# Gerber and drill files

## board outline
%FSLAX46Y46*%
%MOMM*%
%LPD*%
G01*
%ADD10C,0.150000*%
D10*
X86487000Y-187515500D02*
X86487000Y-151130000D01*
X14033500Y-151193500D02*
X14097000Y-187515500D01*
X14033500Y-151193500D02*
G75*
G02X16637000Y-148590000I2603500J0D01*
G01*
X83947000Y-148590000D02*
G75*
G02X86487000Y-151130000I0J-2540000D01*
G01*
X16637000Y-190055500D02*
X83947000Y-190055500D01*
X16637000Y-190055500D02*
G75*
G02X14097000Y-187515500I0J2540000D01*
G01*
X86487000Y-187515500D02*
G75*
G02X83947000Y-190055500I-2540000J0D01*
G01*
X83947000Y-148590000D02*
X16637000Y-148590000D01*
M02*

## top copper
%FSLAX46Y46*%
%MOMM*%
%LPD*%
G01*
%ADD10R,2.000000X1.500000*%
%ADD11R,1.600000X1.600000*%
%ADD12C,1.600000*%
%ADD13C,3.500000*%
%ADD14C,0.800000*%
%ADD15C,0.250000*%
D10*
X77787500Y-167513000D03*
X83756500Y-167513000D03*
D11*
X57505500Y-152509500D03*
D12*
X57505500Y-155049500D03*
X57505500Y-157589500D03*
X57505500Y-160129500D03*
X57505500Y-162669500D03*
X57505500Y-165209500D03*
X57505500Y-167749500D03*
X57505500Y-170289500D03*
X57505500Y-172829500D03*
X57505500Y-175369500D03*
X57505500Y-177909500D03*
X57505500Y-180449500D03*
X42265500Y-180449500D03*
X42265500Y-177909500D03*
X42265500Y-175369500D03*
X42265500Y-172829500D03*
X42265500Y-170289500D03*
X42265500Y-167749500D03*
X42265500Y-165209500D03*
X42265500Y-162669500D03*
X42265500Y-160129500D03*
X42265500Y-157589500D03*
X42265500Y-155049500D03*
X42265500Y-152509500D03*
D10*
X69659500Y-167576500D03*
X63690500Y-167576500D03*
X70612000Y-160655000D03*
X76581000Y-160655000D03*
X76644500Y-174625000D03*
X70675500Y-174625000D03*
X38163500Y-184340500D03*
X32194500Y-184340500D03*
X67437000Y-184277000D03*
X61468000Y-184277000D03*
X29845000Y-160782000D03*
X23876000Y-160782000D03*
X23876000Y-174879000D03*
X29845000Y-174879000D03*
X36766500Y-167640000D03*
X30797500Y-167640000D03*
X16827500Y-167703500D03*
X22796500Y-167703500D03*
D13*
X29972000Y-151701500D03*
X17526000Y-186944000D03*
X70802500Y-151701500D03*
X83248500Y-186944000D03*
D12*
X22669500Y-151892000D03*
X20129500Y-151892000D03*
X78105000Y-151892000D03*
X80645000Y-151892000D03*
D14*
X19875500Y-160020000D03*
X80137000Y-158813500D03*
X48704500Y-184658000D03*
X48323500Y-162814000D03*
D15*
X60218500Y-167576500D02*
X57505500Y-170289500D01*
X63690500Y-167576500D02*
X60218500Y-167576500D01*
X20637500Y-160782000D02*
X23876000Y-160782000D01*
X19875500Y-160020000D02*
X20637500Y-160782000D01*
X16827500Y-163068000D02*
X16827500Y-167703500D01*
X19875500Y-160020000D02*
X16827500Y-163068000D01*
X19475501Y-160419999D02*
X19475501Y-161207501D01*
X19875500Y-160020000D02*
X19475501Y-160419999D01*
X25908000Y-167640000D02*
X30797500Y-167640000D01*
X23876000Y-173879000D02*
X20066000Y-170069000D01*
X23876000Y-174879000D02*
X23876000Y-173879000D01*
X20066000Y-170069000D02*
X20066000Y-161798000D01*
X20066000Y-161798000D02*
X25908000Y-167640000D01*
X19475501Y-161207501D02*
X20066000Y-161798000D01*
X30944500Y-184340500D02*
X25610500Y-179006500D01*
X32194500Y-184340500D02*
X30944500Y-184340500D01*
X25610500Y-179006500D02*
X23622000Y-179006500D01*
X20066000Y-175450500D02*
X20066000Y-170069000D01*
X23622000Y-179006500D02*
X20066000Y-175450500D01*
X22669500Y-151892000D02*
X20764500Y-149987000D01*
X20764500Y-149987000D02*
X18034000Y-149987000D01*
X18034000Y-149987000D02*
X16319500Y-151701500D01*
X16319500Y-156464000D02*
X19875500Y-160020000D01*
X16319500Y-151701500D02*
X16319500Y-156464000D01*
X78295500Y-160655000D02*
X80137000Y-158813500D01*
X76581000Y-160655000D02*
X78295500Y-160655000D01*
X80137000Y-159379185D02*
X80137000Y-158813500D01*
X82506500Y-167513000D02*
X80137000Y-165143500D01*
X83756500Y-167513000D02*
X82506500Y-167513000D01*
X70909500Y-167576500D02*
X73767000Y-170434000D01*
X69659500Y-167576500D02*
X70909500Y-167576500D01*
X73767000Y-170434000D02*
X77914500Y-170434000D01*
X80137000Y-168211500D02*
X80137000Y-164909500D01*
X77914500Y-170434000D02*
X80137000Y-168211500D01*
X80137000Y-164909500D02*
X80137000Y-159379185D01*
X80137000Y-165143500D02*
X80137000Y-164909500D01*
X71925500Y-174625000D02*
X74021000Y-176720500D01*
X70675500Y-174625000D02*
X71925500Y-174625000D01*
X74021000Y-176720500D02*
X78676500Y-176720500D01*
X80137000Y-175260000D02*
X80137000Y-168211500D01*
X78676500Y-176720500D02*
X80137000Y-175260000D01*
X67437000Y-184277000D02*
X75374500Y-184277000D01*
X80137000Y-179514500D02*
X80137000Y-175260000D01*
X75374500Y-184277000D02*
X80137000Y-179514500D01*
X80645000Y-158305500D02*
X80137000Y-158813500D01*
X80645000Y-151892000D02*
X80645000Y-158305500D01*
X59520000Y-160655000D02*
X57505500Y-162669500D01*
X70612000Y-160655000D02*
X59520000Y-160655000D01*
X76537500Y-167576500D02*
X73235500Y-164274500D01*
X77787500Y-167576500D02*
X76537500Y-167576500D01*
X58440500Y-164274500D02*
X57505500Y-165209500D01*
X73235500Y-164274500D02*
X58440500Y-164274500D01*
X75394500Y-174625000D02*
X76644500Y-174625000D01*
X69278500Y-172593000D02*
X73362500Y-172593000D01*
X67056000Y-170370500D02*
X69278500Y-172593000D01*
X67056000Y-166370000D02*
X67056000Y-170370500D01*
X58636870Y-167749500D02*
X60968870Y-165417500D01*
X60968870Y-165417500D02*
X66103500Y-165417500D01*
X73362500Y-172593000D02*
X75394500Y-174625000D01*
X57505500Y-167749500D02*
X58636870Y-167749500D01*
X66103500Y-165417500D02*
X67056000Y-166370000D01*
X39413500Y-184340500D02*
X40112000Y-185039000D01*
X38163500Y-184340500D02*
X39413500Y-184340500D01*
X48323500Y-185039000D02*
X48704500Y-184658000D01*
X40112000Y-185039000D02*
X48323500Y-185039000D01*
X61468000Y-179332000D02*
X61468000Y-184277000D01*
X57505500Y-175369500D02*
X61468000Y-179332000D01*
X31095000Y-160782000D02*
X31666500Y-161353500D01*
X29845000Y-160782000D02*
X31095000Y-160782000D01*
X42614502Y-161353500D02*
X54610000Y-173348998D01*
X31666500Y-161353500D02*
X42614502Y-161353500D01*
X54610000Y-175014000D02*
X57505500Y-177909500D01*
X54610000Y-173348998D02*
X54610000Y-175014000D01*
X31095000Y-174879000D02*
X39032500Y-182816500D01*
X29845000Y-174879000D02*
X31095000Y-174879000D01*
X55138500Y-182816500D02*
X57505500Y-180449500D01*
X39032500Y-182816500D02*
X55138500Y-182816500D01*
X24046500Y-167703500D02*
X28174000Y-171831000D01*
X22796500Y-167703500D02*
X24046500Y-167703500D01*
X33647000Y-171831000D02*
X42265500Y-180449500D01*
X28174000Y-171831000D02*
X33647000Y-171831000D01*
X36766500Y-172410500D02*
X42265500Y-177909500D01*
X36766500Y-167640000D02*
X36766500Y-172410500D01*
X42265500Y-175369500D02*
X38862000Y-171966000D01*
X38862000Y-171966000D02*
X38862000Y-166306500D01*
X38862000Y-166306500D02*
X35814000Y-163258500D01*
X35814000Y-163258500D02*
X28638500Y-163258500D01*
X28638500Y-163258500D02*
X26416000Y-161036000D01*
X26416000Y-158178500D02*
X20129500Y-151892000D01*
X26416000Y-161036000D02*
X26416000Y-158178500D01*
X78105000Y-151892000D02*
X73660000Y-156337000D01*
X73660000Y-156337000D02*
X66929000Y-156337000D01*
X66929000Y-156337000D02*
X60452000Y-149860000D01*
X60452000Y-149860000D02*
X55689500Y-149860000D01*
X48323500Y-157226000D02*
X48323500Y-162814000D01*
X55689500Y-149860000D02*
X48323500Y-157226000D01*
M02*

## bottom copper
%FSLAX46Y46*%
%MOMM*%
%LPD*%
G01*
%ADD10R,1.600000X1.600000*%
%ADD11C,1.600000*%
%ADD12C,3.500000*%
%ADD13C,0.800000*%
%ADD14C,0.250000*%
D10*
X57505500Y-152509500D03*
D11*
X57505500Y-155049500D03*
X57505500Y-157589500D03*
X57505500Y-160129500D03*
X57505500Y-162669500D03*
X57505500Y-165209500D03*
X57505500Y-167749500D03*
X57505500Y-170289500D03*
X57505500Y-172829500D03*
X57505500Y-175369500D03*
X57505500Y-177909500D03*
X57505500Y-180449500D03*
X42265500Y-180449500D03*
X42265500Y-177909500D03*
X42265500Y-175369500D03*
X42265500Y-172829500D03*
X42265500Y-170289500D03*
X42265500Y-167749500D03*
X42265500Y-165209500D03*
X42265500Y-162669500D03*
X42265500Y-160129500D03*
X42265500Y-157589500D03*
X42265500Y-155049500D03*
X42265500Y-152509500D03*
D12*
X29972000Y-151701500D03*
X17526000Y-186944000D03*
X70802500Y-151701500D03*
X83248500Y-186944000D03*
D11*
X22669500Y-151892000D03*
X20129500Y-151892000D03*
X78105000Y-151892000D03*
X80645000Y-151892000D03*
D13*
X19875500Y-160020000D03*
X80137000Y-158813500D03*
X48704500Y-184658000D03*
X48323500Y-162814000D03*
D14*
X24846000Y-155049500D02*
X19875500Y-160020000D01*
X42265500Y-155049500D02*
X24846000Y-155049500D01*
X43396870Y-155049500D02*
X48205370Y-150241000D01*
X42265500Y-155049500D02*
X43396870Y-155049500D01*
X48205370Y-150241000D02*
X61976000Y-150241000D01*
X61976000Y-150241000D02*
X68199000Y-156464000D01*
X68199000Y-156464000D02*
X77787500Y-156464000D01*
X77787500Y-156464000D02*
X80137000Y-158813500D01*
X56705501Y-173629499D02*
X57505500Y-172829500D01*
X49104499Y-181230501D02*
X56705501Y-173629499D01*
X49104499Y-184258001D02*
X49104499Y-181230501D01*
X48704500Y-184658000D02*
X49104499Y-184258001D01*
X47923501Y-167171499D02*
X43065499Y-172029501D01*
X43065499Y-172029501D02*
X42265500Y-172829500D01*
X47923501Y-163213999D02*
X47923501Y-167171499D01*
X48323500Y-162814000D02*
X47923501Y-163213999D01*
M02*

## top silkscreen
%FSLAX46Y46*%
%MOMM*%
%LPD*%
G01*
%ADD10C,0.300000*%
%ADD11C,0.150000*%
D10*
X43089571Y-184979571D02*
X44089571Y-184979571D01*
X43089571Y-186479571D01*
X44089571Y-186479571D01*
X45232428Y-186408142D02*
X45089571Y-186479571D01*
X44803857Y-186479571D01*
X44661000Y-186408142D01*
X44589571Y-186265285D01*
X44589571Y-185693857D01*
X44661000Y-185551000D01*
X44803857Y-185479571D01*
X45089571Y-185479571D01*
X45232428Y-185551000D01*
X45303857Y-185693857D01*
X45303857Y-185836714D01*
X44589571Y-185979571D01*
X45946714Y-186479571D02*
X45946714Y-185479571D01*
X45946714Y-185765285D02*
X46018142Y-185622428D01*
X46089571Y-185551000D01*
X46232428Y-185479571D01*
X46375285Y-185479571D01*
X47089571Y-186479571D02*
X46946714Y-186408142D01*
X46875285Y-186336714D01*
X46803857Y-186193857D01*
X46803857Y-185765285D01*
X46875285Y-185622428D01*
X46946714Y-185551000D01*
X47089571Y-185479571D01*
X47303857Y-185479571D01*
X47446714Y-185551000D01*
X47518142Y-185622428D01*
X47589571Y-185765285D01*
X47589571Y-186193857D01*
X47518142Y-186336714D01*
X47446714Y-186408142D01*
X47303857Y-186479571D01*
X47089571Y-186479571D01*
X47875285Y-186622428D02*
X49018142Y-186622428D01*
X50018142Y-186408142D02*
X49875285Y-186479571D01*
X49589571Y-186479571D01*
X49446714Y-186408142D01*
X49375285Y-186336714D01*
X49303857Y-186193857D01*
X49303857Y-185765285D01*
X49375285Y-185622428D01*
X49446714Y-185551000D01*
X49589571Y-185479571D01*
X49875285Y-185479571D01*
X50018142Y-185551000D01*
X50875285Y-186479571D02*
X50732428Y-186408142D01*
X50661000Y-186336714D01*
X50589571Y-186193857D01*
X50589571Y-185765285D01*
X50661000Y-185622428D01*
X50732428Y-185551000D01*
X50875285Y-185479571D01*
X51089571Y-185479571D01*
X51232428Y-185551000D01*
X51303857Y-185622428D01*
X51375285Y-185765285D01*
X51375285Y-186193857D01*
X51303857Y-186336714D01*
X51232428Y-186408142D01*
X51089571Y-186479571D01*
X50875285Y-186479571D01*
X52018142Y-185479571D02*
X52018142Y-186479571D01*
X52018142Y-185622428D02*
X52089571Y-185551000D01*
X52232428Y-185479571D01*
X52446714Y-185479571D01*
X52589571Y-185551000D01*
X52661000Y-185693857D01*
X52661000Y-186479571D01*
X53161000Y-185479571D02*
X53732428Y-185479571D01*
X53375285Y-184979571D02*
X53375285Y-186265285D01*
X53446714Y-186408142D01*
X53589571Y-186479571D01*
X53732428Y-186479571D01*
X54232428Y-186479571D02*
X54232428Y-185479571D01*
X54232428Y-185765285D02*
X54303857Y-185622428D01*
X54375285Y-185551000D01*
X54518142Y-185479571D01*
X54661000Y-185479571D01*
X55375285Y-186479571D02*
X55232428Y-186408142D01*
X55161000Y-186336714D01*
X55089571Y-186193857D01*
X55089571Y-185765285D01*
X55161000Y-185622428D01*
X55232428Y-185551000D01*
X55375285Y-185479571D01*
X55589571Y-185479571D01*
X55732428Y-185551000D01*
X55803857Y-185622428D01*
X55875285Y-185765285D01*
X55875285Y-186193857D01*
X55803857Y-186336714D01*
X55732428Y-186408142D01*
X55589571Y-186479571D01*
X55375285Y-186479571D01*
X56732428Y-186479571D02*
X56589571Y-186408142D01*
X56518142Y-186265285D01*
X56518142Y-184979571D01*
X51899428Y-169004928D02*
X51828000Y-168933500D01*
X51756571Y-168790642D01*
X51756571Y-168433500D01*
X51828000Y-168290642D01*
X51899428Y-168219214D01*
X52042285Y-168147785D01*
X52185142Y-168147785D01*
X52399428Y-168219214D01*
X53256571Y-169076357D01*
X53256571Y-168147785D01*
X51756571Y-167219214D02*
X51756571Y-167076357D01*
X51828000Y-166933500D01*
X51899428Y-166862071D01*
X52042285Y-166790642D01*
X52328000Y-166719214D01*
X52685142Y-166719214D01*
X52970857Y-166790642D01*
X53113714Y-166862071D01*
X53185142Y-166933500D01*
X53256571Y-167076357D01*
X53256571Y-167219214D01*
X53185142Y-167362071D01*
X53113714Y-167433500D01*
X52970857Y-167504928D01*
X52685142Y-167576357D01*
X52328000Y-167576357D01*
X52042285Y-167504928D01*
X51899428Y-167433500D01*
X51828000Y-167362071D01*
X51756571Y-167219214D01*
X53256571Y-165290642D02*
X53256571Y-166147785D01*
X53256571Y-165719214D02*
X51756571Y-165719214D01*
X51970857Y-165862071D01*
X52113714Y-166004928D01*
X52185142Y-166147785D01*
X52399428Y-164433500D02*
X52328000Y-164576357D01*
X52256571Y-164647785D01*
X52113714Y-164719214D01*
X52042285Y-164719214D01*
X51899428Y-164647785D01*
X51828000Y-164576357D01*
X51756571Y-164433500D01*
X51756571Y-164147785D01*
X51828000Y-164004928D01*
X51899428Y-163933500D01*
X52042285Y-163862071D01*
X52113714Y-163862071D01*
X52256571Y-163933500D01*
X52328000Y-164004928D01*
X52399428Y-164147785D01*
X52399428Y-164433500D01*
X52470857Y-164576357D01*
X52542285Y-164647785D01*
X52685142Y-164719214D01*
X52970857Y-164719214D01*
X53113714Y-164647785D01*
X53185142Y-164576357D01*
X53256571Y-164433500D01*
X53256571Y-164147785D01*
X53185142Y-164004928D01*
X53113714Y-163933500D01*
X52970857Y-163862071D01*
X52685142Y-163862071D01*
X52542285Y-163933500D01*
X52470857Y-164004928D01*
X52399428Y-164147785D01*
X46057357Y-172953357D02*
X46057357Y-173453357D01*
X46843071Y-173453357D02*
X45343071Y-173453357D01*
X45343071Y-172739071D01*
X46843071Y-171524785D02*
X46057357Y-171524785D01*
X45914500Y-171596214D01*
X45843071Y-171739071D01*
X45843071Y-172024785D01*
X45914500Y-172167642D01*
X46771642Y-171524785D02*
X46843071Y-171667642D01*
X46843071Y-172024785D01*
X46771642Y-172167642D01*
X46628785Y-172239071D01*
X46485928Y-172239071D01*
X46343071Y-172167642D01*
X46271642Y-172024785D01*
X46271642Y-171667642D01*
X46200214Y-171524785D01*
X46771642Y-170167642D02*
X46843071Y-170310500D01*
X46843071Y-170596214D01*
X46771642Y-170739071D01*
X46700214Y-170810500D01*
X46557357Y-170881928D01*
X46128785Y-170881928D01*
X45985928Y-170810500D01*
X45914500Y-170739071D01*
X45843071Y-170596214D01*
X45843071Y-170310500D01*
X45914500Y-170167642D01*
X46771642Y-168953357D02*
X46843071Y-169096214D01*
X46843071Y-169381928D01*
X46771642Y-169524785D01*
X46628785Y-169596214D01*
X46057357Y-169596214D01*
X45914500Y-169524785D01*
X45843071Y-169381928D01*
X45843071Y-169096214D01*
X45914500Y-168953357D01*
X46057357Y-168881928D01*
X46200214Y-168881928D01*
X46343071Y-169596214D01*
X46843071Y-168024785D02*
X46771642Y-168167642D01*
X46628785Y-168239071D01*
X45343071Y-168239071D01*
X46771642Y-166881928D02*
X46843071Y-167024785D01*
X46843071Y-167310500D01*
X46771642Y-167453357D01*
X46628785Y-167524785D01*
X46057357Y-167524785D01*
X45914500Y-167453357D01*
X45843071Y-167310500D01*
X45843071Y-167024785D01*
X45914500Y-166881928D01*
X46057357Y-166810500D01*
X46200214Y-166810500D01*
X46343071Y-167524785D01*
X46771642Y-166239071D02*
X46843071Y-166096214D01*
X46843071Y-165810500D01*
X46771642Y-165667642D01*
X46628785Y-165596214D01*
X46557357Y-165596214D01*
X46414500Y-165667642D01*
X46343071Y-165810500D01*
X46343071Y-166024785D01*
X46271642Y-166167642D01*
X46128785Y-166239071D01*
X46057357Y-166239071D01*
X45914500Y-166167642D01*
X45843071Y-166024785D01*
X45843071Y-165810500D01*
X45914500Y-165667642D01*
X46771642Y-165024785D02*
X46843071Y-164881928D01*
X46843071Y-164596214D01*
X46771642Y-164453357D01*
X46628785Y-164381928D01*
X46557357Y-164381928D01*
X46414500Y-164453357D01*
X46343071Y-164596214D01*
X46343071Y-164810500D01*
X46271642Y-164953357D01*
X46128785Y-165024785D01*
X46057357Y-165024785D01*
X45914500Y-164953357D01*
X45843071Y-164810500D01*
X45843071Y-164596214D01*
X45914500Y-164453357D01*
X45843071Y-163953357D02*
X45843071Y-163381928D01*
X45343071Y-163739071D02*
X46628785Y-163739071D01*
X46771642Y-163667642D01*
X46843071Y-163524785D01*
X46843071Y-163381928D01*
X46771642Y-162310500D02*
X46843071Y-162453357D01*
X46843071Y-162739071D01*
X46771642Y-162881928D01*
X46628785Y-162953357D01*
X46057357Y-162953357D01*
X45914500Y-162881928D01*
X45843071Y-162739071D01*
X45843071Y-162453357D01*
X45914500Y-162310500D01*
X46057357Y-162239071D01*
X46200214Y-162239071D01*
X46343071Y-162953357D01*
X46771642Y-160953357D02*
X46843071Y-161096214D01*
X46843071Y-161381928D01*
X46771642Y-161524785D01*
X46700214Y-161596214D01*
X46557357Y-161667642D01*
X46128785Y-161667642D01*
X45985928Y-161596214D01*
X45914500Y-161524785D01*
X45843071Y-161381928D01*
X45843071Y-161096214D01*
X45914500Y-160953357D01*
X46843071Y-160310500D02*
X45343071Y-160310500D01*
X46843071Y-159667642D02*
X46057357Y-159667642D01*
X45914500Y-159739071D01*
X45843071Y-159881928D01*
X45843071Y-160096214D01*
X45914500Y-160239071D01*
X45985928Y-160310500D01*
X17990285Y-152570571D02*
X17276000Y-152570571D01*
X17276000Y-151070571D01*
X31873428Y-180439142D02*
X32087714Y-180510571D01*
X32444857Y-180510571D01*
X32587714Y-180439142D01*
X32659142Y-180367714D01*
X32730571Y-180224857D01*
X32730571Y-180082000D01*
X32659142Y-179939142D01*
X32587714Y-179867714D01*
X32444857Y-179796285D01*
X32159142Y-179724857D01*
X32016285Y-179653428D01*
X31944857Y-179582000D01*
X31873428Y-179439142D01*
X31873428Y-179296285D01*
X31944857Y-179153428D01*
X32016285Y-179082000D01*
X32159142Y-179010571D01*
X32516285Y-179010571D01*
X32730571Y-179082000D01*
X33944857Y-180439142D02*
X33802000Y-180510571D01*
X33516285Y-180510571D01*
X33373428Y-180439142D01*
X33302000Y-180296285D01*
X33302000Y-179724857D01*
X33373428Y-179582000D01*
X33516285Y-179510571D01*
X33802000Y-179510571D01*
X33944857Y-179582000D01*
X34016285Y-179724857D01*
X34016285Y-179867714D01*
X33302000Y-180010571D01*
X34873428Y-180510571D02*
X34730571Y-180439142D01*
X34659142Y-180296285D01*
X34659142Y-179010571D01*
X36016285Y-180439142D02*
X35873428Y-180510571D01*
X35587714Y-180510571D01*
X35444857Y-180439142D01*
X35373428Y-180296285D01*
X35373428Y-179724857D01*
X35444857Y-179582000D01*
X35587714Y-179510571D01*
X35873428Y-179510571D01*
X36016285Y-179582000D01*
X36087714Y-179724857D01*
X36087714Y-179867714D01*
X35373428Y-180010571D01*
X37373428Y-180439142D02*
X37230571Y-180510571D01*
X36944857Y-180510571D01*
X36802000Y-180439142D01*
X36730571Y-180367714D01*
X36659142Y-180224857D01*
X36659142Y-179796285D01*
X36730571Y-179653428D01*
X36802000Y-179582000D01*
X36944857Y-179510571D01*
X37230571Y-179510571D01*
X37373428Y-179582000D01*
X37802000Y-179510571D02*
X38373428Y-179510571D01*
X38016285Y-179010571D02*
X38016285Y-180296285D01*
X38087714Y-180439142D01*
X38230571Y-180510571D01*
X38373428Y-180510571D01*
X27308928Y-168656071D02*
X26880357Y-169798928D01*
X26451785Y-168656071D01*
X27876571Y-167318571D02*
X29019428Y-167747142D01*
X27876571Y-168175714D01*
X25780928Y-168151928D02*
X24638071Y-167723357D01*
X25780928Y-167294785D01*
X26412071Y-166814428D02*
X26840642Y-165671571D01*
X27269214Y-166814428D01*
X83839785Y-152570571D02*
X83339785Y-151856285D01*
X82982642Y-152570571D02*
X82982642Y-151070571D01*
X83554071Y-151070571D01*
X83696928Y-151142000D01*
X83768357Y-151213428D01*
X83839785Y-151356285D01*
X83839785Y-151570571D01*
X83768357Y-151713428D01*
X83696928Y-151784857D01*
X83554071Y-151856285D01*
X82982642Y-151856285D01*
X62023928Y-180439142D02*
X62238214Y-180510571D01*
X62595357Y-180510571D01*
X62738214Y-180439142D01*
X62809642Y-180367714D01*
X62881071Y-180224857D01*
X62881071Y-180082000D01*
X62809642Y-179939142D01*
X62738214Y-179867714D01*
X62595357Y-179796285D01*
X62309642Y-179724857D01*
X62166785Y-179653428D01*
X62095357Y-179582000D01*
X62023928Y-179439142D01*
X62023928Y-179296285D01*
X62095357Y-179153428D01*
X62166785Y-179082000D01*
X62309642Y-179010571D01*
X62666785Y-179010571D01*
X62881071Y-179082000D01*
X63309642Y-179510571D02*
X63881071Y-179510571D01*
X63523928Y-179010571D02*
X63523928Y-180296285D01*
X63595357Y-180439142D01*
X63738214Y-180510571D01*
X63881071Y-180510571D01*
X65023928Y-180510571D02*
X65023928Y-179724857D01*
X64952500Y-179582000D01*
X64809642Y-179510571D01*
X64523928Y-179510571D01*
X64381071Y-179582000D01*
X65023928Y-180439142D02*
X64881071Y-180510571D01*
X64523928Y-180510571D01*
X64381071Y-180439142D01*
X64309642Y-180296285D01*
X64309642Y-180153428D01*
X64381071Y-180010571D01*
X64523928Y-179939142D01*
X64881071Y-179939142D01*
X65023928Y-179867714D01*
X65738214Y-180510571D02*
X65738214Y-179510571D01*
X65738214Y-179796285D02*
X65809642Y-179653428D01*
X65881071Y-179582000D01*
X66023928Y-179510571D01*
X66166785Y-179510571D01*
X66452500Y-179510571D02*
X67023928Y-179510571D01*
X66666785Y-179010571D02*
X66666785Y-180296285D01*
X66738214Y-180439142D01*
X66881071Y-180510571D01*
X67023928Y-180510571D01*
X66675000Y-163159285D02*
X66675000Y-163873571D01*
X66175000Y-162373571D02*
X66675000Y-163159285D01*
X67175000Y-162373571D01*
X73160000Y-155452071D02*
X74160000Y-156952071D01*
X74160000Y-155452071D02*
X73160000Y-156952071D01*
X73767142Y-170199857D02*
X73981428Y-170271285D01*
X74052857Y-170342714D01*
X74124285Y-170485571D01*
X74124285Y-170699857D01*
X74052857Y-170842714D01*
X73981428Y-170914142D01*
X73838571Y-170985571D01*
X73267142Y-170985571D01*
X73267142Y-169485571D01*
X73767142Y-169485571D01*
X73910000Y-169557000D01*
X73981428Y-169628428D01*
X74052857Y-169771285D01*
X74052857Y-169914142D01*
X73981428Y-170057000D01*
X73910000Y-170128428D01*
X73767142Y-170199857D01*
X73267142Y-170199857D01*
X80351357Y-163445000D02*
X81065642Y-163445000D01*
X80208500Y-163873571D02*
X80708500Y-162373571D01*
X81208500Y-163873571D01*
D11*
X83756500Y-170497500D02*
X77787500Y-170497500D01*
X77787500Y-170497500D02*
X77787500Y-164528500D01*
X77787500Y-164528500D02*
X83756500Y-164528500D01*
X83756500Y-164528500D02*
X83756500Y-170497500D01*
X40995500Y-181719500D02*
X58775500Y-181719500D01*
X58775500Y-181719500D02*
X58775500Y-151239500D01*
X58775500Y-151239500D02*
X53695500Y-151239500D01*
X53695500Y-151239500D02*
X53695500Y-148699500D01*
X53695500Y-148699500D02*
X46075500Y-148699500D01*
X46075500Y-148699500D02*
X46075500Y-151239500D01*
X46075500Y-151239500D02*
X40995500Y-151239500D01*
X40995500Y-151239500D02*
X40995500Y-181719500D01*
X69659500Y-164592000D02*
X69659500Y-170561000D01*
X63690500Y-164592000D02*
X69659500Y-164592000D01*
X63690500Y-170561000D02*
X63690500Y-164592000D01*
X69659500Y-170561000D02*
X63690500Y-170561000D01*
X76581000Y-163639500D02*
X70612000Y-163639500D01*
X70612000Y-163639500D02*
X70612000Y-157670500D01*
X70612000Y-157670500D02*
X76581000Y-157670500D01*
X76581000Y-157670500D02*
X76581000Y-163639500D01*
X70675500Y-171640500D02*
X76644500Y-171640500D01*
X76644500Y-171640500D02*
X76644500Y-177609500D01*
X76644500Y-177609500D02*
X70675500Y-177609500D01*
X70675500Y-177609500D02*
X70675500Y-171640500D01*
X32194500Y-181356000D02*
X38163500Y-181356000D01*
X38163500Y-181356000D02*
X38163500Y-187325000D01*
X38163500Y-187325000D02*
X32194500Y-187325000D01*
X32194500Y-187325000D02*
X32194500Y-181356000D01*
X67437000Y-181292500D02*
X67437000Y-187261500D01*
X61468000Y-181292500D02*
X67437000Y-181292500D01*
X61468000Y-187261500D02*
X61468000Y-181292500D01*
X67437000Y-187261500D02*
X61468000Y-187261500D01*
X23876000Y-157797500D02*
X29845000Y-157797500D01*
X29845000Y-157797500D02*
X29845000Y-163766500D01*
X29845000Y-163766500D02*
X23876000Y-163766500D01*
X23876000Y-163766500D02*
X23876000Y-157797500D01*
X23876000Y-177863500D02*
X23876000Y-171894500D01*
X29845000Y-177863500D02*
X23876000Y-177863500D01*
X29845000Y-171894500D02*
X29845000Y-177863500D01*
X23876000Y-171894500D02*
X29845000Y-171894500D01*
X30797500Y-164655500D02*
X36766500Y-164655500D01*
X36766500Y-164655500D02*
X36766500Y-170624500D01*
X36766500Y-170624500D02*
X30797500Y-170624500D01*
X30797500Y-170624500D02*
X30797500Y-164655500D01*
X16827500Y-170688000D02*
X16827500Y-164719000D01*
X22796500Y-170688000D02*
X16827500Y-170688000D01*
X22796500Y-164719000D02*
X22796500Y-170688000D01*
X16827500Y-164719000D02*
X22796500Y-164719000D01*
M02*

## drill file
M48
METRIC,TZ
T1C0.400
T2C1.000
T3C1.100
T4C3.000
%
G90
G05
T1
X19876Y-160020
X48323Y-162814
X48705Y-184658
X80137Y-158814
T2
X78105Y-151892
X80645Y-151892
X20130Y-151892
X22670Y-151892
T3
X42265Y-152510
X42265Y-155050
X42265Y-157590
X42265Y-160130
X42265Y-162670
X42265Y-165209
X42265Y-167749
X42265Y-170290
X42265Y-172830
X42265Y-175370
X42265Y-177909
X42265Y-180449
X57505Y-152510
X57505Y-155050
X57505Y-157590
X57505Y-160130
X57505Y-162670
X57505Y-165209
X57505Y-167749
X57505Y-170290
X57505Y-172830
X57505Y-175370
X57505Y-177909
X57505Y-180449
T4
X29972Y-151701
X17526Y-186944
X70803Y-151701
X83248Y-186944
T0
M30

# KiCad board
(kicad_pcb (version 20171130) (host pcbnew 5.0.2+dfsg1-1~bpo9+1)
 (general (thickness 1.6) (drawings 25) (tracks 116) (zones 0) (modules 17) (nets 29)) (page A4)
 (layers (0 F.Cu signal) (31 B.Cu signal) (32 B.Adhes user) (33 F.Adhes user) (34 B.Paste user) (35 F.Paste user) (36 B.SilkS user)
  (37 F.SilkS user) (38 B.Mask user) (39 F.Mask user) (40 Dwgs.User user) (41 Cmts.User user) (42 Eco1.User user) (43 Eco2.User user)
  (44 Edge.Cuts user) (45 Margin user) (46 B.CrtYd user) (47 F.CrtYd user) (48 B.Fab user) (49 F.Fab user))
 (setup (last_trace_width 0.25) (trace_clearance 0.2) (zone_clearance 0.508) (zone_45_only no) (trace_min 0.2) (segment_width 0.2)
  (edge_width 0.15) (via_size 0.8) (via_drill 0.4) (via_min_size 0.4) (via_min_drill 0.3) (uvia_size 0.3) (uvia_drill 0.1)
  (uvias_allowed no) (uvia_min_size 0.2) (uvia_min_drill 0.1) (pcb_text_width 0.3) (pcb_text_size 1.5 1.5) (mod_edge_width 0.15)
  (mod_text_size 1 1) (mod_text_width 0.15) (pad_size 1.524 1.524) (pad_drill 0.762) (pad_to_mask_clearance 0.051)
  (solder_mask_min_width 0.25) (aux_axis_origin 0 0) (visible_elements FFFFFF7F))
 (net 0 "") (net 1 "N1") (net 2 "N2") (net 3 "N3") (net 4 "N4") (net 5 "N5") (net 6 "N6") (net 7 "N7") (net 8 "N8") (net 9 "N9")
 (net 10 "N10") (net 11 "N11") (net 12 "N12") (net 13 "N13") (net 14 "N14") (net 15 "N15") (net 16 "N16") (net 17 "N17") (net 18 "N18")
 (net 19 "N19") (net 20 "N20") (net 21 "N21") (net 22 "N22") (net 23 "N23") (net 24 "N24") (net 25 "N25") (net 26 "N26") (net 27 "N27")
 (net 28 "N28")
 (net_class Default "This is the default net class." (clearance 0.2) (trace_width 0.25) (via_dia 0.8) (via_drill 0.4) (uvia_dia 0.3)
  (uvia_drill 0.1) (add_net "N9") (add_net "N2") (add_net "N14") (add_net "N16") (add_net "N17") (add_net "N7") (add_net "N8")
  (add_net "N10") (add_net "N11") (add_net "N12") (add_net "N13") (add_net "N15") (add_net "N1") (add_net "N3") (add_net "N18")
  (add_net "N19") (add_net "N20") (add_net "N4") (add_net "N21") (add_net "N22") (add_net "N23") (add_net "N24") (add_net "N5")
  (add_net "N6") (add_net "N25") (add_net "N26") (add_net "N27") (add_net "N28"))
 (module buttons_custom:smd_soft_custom (layer F.Cu) (at 80.772 167.513 180)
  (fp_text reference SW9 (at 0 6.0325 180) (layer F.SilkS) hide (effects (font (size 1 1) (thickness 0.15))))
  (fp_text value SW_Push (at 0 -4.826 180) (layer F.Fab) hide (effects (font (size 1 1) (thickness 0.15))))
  (fp_line (start -2.9845 -2.9845) (end 2.9845 -2.9845) (layer F.SilkS) (width 0.15))
  (fp_line (start 2.9845 -2.9845) (end 2.9845 2.9845) (layer F.SilkS) (width 0.15))
  (fp_line (start 2.9845 2.9845) (end -2.9845 2.9845) (layer F.SilkS) (width 0.15))
  (fp_line (start -2.9845 2.9845) (end -2.9845 -2.9845) (layer F.SilkS) (width 0.15))
  (pad 1 smd rect (at 2.9845 0 270) (size 1.5 2) (layers F.Cu F.Paste F.Mask) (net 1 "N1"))
  (pad 2 smd rect (at -2.9845 0 270) (size 1.5 2) (layers F.Cu F.Paste F.Mask) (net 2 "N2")))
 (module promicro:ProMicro (layer B.Cu) (at 49.8855 166.4795 270)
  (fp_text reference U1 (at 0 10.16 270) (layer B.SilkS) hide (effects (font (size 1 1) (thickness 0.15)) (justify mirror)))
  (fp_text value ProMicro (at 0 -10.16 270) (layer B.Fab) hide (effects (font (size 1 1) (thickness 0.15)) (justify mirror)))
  (fp_line (start 15.24 8.89) (end 15.24 -8.89) (layer F.SilkS) (width 0.15))
  (fp_line (start 15.24 -8.89) (end -15.24 -8.89) (layer F.SilkS) (width 0.15))
  (fp_line (start -15.24 -8.89) (end -15.24 -3.81) (layer F.SilkS) (width 0.15))
  (fp_line (start -15.24 -3.81) (end -17.78 -3.81) (layer F.SilkS) (width 0.15))
  (fp_line (start -17.78 -3.81) (end -17.78 3.81) (layer F.SilkS) (width 0.15))
  (fp_line (start -17.78 3.81) (end -15.24 3.81) (layer F.SilkS) (width 0.15))
  (fp_line (start -15.24 3.81) (end -15.24 8.89) (layer F.SilkS) (width 0.15))
  (fp_line (start -15.24 8.89) (end 15.24 8.89) (layer F.SilkS) (width 0.15))
  (pad 1 thru_hole rect (at -13.97 -7.62 270) (size 1.6 1.6) (drill 1.1) (layers *.Cu *.Mask B.SilkS) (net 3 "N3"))
  (pad 2 thru_hole circle (at -11.43 -7.62 270) (size 1.6 1.6) (drill 1.1) (layers *.Cu *.Mask B.SilkS) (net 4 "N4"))
  (pad 3 thru_hole circle (at -8.89 -7.62 270) (size 1.6 1.6) (drill 1.1) (layers *.Cu *.Mask B.SilkS) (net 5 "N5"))
  (pad 4 thru_hole circle (at -6.35 -7.62 270) (size 1.6 1.6) (drill 1.1) (layers *.Cu *.Mask B.SilkS) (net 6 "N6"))
  (pad 5 thru_hole circle (at -3.81 -7.62 270) (size 1.6 1.6) (drill 1.1) (layers *.Cu *.Mask B.SilkS) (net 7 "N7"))
  (pad 6 thru_hole circle (at -1.27 -7.62 270) (size 1.6 1.6) (drill 1.1) (layers *.Cu *.Mask B.SilkS) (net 1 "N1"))
  (pad 7 thru_hole circle (at 1.27 -7.62 270) (size 1.6 1.6) (drill 1.1) (layers *.Cu *.Mask B.SilkS) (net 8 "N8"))
  (pad 8 thru_hole circle (at 3.81 -7.62 270) (size 1.6 1.6) (drill 1.1) (layers *.Cu *.Mask B.SilkS) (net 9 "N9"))
  (pad 9 thru_hole circle (at 6.35 -7.62 270) (size 1.6 1.6) (drill 1.1) (layers *.Cu *.Mask B.SilkS) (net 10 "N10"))
  (pad 10 thru_hole circle (at 8.89 -7.62 270) (size 1.6 1.6) (drill 1.1) (layers *.Cu *.Mask B.SilkS) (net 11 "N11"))
  (pad 11 thru_hole circle (at 11.43 -7.62 270) (size 1.6 1.6) (drill 1.1) (layers *.Cu *.Mask B.SilkS) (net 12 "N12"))
  (pad 12 thru_hole circle (at 13.97 -7.62 270) (size 1.6 1.6) (drill 1.1) (layers *.Cu *.Mask B.SilkS) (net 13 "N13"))
  (pad 13 thru_hole circle (at 13.97 7.62 270) (size 1.6 1.6) (drill 1.1) (layers *.Cu *.Mask B.SilkS) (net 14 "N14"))
  (pad 14 thru_hole circle (at 11.43 7.62 270) (size 1.6 1.6) (drill 1.1) (layers *.Cu *.Mask B.SilkS) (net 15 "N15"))
  (pad 15 thru_hole circle (at 8.89 7.62 270) (size 1.6 1.6) (drill 1.1) (layers *.Cu *.Mask B.SilkS) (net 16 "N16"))
  (pad 16 thru_hole circle (at 6.35 7.62 270) (size 1.6 1.6) (drill 1.1) (layers *.Cu *.Mask B.SilkS) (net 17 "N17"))
  (pad 17 thru_hole circle (at 3.81 7.62 270) (size 1.6 1.6) (drill 1.1) (layers *.Cu *.Mask B.SilkS) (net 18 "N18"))
  (pad 18 thru_hole circle (at 1.27 7.62 270) (size 1.6 1.6) (drill 1.1) (layers *.Cu *.Mask B.SilkS) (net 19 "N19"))
  (pad 19 thru_hole circle (at -1.27 7.62 270) (size 1.6 1.6) (drill 1.1) (layers *.Cu *.Mask B.SilkS) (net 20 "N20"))
  (pad 20 thru_hole circle (at -3.81 7.62 270) (size 1.6 1.6) (drill 1.1) (layers *.Cu *.Mask B.SilkS) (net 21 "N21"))
  (pad 21 thru_hole circle (at -6.35 7.62 270) (size 1.6 1.6) (drill 1.1) (layers *.Cu *.Mask B.SilkS) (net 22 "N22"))
  (pad 22 thru_hole circle (at -8.89 7.62 270) (size 1.6 1.6) (drill 1.1) (layers *.Cu *.Mask B.SilkS) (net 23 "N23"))
  (pad 23 thru_hole circle (at -11.43 7.62 270) (size 1.6 1.6) (drill 1.1) (layers *.Cu *.Mask B.SilkS) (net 2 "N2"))
  (pad 24 thru_hole circle (at -13.97 7.62 270) (size 1.6 1.6) (drill 1.1) (layers *.Cu *.Mask B.SilkS) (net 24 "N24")))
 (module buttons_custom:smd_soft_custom (layer F.Cu) (at 66.675 167.5765 180)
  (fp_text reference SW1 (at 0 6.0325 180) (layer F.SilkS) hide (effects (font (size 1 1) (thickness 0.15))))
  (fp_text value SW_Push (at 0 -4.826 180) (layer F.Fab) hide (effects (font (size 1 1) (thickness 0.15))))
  (fp_line (start -2.9845 2.9845) (end -2.9845 -2.9845) (layer F.SilkS) (width 0.15))
  (fp_line (start 2.9845 2.9845) (end -2.9845 2.9845) (layer F.SilkS) (width 0.15))
  (fp_line (start 2.9845 -2.9845) (end 2.9845 2.9845) (layer F.SilkS) (width 0.15))
  (fp_line (start -2.9845 -2.9845) (end 2.9845 -2.9845) (layer F.SilkS) (width 0.15))
  (pad 2 smd rect (at -2.9845 0 270) (size 1.5 2) (layers F.Cu F.Paste F.Mask) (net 2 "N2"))
  (pad 1 smd rect (at 2.9845 0 270) (size 1.5 2) (layers F.Cu F.Paste F.Mask) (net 9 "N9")))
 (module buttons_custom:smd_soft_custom (layer F.Cu) (at 73.5965 160.655 180)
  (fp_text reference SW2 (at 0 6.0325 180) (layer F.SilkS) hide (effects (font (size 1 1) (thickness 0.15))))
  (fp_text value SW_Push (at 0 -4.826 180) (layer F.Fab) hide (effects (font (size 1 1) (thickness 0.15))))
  (fp_line (start -2.9845 -2.9845) (end 2.9845 -2.9845) (layer F.SilkS) (width 0.15))
  (fp_line (start 2.9845 -2.9845) (end 2.9845 2.9845) (layer F.SilkS) (width 0.15))
  (fp_line (start 2.9845 2.9845) (end -2.9845 2.9845) (layer F.SilkS) (width 0.15))
  (fp_line (start -2.9845 2.9845) (end -2.9845 -2.9845) (layer F.SilkS) (width 0.15))
  (pad 1 smd rect (at 2.9845 0 270) (size 1.5 2) (layers F.Cu F.Paste F.Mask) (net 7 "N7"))
  (pad 2 smd rect (at -2.9845 0 270) (size 1.5 2) (layers F.Cu F.Paste F.Mask) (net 2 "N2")))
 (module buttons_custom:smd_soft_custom (layer F.Cu) (at 73.66 174.625)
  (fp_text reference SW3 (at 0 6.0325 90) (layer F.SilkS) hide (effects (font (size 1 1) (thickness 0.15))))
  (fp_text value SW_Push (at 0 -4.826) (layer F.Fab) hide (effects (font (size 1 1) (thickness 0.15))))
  (fp_line (start -2.9845 -2.9845) (end 2.9845 -2.9845) (layer F.SilkS) (width 0.15))
  (fp_line (start 2.9845 -2.9845) (end 2.9845 2.9845) (layer F.SilkS) (width 0.15))
  (fp_line (start 2.9845 2.9845) (end -2.9845 2.9845) (layer F.SilkS) (width 0.15))
  (fp_line (start -2.9845 2.9845) (end -2.9845 -2.9845) (layer F.SilkS) (width 0.15))
  (pad 1 smd rect (at 2.9845 0 90) (size 1.5 2) (layers F.Cu F.Paste F.Mask) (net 8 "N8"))
  (pad 2 smd rect (at -2.9845 0 90) (size 1.5 2) (layers F.Cu F.Paste F.Mask) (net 2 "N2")))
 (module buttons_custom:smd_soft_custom (layer F.Cu) (at 35.179 184.3405)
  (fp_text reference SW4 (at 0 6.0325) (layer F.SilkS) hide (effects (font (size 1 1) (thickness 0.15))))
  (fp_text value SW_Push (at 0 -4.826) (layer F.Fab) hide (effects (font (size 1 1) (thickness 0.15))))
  (fp_line (start -2.9845 -2.9845) (end 2.9845 -2.9845) (layer F.SilkS) (width 0.15))
  (fp_line (start 2.9845 -2.9845) (end 2.9845 2.9845) (layer F.SilkS) (width 0.15))
  (fp_line (start 2.9845 2.9845) (end -2.9845 2.9845) (layer F.SilkS) (width 0.15))
  (fp_line (start -2.9845 2.9845) (end -2.9845 -2.9845) (layer F.SilkS) (width 0.15))
  (pad 1 smd rect (at 2.9845 0 90) (size 1.5 2) (layers F.Cu F.Paste F.Mask) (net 10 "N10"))
  (pad 2 smd rect (at -2.9845 0 90) (size 1.5 2) (layers F.Cu F.Paste F.Mask) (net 2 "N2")))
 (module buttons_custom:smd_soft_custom (layer F.Cu) (at 64.4525 184.277 180)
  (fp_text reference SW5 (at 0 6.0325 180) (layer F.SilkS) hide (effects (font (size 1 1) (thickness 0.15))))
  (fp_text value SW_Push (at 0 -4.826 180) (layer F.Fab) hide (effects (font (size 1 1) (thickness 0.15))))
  (fp_line (start -2.9845 2.9845) (end -2.9845 -2.9845) (layer F.SilkS) (width 0.15))
  (fp_line (start 2.9845 2.9845) (end -2.9845 2.9845) (layer F.SilkS) (width 0.15))
  (fp_line (start 2.9845 -2.9845) (end 2.9845 2.9845) (layer F.SilkS) (width 0.15))
  (fp_line (start -2.9845 -2.9845) (end 2.9845 -2.9845) (layer F.SilkS) (width 0.15))
  (pad 2 smd rect (at -2.9845 0 270) (size 1.5 2) (layers F.Cu F.Paste F.Mask) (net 2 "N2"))
  (pad 1 smd rect (at 2.9845 0 270) (size 1.5 2) (layers F.Cu F.Paste F.Mask) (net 11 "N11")))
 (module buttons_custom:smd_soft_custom (layer F.Cu) (at 26.8605 160.782)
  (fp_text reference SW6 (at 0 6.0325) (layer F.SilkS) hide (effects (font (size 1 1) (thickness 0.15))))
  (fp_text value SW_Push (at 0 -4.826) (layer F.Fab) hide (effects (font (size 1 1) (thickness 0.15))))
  (fp_line (start -2.9845 -2.9845) (end 2.9845 -2.9845) (layer F.SilkS) (width 0.15))
  (fp_line (start 2.9845 -2.9845) (end 2.9845 2.9845) (layer F.SilkS) (width 0.15))
  (fp_line (start 2.9845 2.9845) (end -2.9845 2.9845) (layer F.SilkS) (width 0.15))
  (fp_line (start -2.9845 2.9845) (end -2.9845 -2.9845) (layer F.SilkS) (width 0.15))
  (pad 1 smd rect (at 2.9845 0 90) (size 1.5 2) (layers F.Cu F.Paste F.Mask) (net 12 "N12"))
  (pad 2 smd rect (at -2.9845 0 90) (size 1.5 2) (layers F.Cu F.Paste F.Mask) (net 2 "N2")))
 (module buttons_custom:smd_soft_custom (layer F.Cu) (at 26.8605 174.879)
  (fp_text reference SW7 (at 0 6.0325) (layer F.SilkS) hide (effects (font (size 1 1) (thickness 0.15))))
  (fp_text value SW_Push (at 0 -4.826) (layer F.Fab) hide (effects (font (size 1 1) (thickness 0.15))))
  (fp_line (start -2.9845 2.9845) (end -2.9845 -2.9845) (layer F.SilkS) (width 0.15))
  (fp_line (start 2.9845 2.9845) (end -2.9845 2.9845) (layer F.SilkS) (width 0.15))
  (fp_line (start 2.9845 -2.9845) (end 2.9845 2.9845) (layer F.SilkS) (width 0.15))
  (fp_line (start -2.9845 -2.9845) (end 2.9845 -2.9845) (layer F.SilkS) (width 0.15))
  (pad 2 smd rect (at -2.9845 0 90) (size 1.5 2) (layers F.Cu F.Paste F.Mask) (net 2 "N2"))
  (pad 1 smd rect (at 2.9845 0 90) (size 1.5 2) (layers F.Cu F.Paste F.Mask) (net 13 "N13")))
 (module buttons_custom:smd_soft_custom (layer F.Cu) (at 33.782 167.64)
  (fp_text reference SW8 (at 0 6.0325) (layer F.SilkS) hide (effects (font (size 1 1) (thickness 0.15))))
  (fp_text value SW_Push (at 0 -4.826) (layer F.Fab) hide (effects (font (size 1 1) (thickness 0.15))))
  (fp_line (start -2.9845 -2.9845) (end 2.9845 -2.9845) (layer F.SilkS) (width 0.15))
  (fp_line (start 2.9845 -2.9845) (end 2.9845 2.9845) (layer F.SilkS) (width 0.15))
  (fp_line (start 2.9845 2.9845) (end -2.9845 2.9845) (layer F.SilkS) (width 0.15))
  (fp_line (start -2.9845 2.9845) (end -2.9845 -2.9845) (layer F.SilkS) (width 0.15))
  (pad 1 smd rect (at 2.9845 0 90) (size 1.5 2) (layers F.Cu F.Paste F.Mask) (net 15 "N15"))
  (pad 2 smd rect (at -2.9845 0 90) (size 1.5 2) (layers F.Cu F.Paste F.Mask) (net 2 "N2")))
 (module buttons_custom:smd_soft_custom (layer F.Cu) (at 19.812 167.7035)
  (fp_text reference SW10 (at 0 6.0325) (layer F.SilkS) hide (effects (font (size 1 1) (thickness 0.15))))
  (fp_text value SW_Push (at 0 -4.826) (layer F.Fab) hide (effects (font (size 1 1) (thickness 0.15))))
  (fp_line (start -2.9845 2.9845) (end -2.9845 -2.9845) (layer F.SilkS) (width 0.15))
  (fp_line (start 2.9845 2.9845) (end -2.9845 2.9845) (layer F.SilkS) (width 0.15))
  (fp_line (start 2.9845 -2.9845) (end 2.9845 2.9845) (layer F.SilkS) (width 0.15))
  (fp_line (start -2.9845 -2.9845) (end 2.9845 -2.9845) (layer F.SilkS) (width 0.15))
  (pad 2 smd rect (at -2.9845 0 90) (size 1.5 2) (layers F.Cu F.Paste F.Mask) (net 2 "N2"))
  (pad 1 smd rect (at 2.9845 0 90) (size 1.5 2) (layers F.Cu F.Paste F.Mask) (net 14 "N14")))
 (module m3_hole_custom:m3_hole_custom (layer F.Cu) (at 29.972 151.7015)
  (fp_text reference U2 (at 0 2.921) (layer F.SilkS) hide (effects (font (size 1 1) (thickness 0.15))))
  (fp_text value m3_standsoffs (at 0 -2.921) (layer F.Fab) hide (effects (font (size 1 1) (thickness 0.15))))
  (pad 1 thru_hole circle (at 0 0) (size 3.5 3.5) (drill 3) (layers *.Cu *.Mask) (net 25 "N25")))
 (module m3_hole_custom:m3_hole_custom (layer F.Cu) (at 17.526 186.944)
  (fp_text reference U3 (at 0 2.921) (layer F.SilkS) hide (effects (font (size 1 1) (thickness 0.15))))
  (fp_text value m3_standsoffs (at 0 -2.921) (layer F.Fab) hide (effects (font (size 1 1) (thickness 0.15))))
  (pad 1 thru_hole circle (at 0 0) (size 3.5 3.5) (drill 3) (layers *.Cu *.Mask) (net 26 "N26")))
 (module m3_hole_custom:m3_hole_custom (layer F.Cu) (at 70.8025 151.7015)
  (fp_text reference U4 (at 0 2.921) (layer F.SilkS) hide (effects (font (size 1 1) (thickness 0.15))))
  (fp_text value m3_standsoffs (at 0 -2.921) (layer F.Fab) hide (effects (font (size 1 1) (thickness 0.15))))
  (pad 1 thru_hole circle (at 0 0) (size 3.5 3.5) (drill 3) (layers *.Cu *.Mask) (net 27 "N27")))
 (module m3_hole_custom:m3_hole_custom (layer F.Cu) (at 83.2485 186.944)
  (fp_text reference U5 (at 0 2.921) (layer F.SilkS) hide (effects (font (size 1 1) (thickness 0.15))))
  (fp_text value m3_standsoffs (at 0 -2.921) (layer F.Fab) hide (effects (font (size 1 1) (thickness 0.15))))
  (pad 1 thru_hole circle (at 0 0) (size 3.5 3.5) (drill 3) (layers *.Cu *.Mask) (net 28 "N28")))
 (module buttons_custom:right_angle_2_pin (layer F.Cu) (at 21.3995 151.892)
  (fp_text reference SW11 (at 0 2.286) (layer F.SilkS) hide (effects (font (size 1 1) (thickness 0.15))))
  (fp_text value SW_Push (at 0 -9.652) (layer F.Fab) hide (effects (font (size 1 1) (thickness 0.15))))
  (pad 2 thru_hole circle (at 1.27 0) (size 1.6 1.6) (drill 1) (layers *.Cu *.Mask) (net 2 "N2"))
  (pad 1 thru_hole circle (at -1.27 0) (size 1.6 1.6) (drill 1) (layers *.Cu *.Mask) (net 16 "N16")))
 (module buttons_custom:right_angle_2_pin (layer F.Cu) (at 79.375 151.892)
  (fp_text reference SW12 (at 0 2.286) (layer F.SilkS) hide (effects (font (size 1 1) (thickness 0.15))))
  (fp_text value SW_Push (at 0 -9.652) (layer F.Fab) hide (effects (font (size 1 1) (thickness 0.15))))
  (pad 1 thru_hole circle (at -1.27 0) (size 1.6 1.6) (drill 1) (layers *.Cu *.Mask) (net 17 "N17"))
  (pad 2 thru_hole circle (at 1.27 0) (size 1.6 1.6) (drill 1) (layers *.Cu *.Mask) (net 2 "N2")))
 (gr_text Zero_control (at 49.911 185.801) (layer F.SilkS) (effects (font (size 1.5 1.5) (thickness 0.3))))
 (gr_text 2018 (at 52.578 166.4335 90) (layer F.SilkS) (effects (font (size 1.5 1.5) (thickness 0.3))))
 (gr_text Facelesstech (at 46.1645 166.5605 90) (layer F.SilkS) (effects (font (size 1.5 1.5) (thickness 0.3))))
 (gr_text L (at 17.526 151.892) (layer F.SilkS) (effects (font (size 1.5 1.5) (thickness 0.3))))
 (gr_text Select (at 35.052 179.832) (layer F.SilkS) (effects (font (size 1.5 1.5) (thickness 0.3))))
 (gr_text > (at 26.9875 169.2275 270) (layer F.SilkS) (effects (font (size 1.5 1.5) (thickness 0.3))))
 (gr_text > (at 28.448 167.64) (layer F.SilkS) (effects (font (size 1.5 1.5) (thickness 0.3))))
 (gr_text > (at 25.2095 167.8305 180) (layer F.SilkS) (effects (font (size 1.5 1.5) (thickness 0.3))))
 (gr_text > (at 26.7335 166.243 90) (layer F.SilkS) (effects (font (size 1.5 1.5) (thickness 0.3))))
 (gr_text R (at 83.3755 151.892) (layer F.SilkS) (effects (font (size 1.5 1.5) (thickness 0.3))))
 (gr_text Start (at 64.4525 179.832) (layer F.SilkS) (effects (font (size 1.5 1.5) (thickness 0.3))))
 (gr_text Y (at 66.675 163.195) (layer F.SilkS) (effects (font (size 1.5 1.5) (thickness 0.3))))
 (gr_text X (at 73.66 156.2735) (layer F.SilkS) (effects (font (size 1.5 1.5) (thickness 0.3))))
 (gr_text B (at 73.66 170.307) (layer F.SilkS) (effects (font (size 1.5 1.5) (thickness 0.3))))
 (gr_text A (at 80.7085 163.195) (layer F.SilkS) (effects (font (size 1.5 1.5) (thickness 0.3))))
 (gr_line (start 86.487 187.5155) (end 86.487 151.13) (layer Edge.Cuts) (width 0.15))
 (gr_line (start 14.0335 151.1935) (end 14.097 187.5155) (layer Edge.Cuts) (width 0.15))
 (gr_arc (start 16.637 151.1935) (end 16.637 148.59) (angle -90) (layer Edge.Cuts) (width 0.15))
 (gr_arc (start 83.947 151.13) (end 86.487 151.13) (angle -90) (layer Edge.Cuts) (width 0.15))
 (gr_line (start 16.637 190.0555) (end 83.947 190.0555) (layer Edge.Cuts) (width 0.15))
 (gr_arc (start 16.637 187.5155) (end 14.097 187.5155) (angle -90) (layer Edge.Cuts) (width 0.15))
 (gr_arc (start 83.947 187.5155) (end 83.947 190.0555) (angle -90) (layer Edge.Cuts) (width 0.15))
 (gr_line (start 83.947 148.59) (end 16.637 148.59) (layer Edge.Cuts) (width 0.15))
 (segment (start 60.2185 167.5765) (end 57.5055 170.2895) (width 0.25) (layer F.Cu) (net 9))
 (segment (start 63.6905 167.5765) (end 60.2185 167.5765) (width 0.25) (layer F.Cu) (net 9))
 (via (at 19.8755 160.02) (size 0.8) (drill 0.4) (layers F.Cu B.Cu) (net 2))
 (segment (start 24.846 155.0495) (end 19.8755 160.02) (width 0.25) (layer B.Cu) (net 2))
 (segment (start 42.2655 155.0495) (end 24.846 155.0495) (width 0.25) (layer B.Cu) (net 2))
 (segment (start 20.6375 160.782) (end 23.876 160.782) (width 0.25) (layer F.Cu) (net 2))
 (segment (start 19.8755 160.02) (end 20.6375 160.782) (width 0.25) (layer F.Cu) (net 2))
 (segment (start 16.8275 163.068) (end 16.8275 167.7035) (width 0.25) (layer F.Cu) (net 2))
 (segment (start 19.8755 160.02) (end 16.8275 163.068) (width 0.25) (layer F.Cu) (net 2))
 (segment (start 19.475501 160.419999) (end 19.475501 161.207501) (width 0.25) (layer F.Cu) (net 2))
 (segment (start 19.8755 160.02) (end 19.475501 160.419999) (width 0.25) (layer F.Cu) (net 2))
 (segment (start 25.908 167.64) (end 30.7975 167.64) (width 0.25) (layer F.Cu) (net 2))
 (segment (start 23.876 173.879) (end 20.066 170.069) (width 0.25) (layer F.Cu) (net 2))
 (segment (start 23.876 174.879) (end 23.876 173.879) (width 0.25) (layer F.Cu) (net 2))
 (segment (start 20.066 170.069) (end 20.066 161.798) (width 0.25) (layer F.Cu) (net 2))
 (segment (start 20.066 161.798) (end 25.908 167.64) (width 0.25) (layer F.Cu) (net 2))
 (segment (start 19.475501 161.207501) (end 20.066 161.798) (width 0.25) (layer F.Cu) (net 2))
 (segment (start 30.9445 184.3405) (end 25.6105 179.0065) (width 0.25) (layer F.Cu) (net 2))
 (segment (start 32.1945 184.3405) (end 30.9445 184.3405) (width 0.25) (layer F.Cu) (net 2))
 (segment (start 25.6105 179.0065) (end 23.622 179.0065) (width 0.25) (layer F.Cu) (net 2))
 (segment (start 20.066 175.4505) (end 20.066 170.069) (width 0.25) (layer F.Cu) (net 2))
 (segment (start 23.622 179.0065) (end 20.066 175.4505) (width 0.25) (layer F.Cu) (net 2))
 (segment (start 22.6695 151.892) (end 20.7645 149.987) (width 0.25) (layer F.Cu) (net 2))
 (segment (start 20.7645 149.987) (end 18.034 149.987) (width 0.25) (layer F.Cu) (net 2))
 (segment (start 18.034 149.987) (end 16.3195 151.7015) (width 0.25) (layer F.Cu) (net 2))
 (segment (start 16.3195 156.464) (end 19.8755 160.02) (width 0.25) (layer F.Cu) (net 2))
 (segment (start 16.3195 151.7015) (end 16.3195 156.464) (width 0.25) (layer F.Cu) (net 2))
 (segment (start 43.39687 155.0495) (end 48.20537 150.241) (width 0.25) (layer B.Cu) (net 2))
 (segment (start 42.2655 155.0495) (end 43.39687 155.0495) (width 0.25) (layer B.Cu) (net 2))
 (segment (start 48.20537 150.241) (end 61.976 150.241) (width 0.25) (layer B.Cu) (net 2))
 (segment (start 61.976 150.241) (end 68.199 156.464) (width 0.25) (layer B.Cu) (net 2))
 (segment (start 68.199 156.464) (end 77.7875 156.464) (width 0.25) (layer B.Cu) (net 2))
 (segment (start 77.7875 156.464) (end 80.137 158.8135) (width 0.25) (layer B.Cu) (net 2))
 (via (at 80.137 158.8135) (size 0.8) (drill 0.4) (layers F.Cu B.Cu) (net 2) (status 1000000))
 (segment (start 78.2955 160.655) (end 80.137 158.8135) (width 0.25) (layer F.Cu) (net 2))
 (segment (start 76.581 160.655) (end 78.2955 160.655) (width 0.25) (layer F.Cu) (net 2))
 (segment (start 80.137 159.379185) (end 80.137 158.8135) (width 0.25) (layer F.Cu) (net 2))
 (segment (start 82.5065 167.513) (end 80.137 165.1435) (width 0.25) (layer F.Cu) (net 2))
 (segment (start 83.7565 167.513) (end 82.5065 167.513) (width 0.25) (layer F.Cu) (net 2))
 (segment (start 70.9095 167.5765) (end 73.767 170.434) (width 0.25) (layer F.Cu) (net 2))
 (segment (start 69.6595 167.5765) (end 70.9095 167.5765) (width 0.25) (layer F.Cu) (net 2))
 (segment (start 73.767 170.434) (end 77.9145 170.434) (width 0.25) (layer F.Cu) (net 2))
 (segment (start 80.137 168.2115) (end 80.137 164.9095) (width 0.25) (layer F.Cu) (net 2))
 (segment (start 77.9145 170.434) (end 80.137 168.2115) (width 0.25) (layer F.Cu) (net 2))
 (segment (start 80.137 164.9095) (end 80.137 159.379185) (width 0.25) (layer F.Cu) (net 2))
 (segment (start 80.137 165.1435) (end 80.137 164.9095) (width 0.25) (layer F.Cu) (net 2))
 (segment (start 71.9255 174.625) (end 74.021 176.7205) (width 0.25) (layer F.Cu) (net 2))
 (segment (start 70.6755 174.625) (end 71.9255 174.625) (width 0.25) (layer F.Cu) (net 2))
 (segment (start 74.021 176.7205) (end 78.6765 176.7205) (width 0.25) (layer F.Cu) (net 2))
 (segment (start 80.137 175.26) (end 80.137 168.2115) (width 0.25) (layer F.Cu) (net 2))
 (segment (start 78.6765 176.7205) (end 80.137 175.26) (width 0.25) (layer F.Cu) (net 2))
 (segment (start 67.437 184.277) (end 75.3745 184.277) (width 0.25) (layer F.Cu) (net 2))
 (segment (start 80.137 179.5145) (end 80.137 175.26) (width 0.25) (layer F.Cu) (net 2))
 (segment (start 75.3745 184.277) (end 80.137 179.5145) (width 0.25) (layer F.Cu) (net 2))
 (segment (start 80.645 158.3055) (end 80.137 158.8135) (width 0.25) (layer F.Cu) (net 2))
 (segment (start 80.645 151.892) (end 80.645 158.3055) (width 0.25) (layer F.Cu) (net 2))
 (segment (start 59.52 160.655) (end 57.5055 162.6695) (width 0.25) (layer F.Cu) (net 7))
 (segment (start 70.612 160.655) (end 59.52 160.655) (width 0.25) (layer F.Cu) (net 7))
 (segment (start 76.5375 167.5765) (end 73.2355 164.2745) (width 0.25) (layer F.Cu) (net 1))
 (segment (start 77.7875 167.5765) (end 76.5375 167.5765) (width 0.25) (layer F.Cu) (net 1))
 (segment (start 58.4405 164.2745) (end 57.5055 165.2095) (width 0.25) (layer F.Cu) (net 1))
 (segment (start 73.2355 164.2745) (end 58.4405 164.2745) (width 0.25) (layer F.Cu) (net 1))
 (segment (start 75.3945 174.625) (end 76.6445 174.625) (width 0.25) (layer F.Cu) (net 8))
 (segment (start 69.2785 172.593) (end 73.3625 172.593) (width 0.25) (layer F.Cu) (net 8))
 (segment (start 67.056 170.3705) (end 69.2785 172.593) (width 0.25) (layer F.Cu) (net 8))
 (segment (start 67.056 166.37) (end 67.056 170.3705) (width 0.25) (layer F.Cu) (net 8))
 (segment (start 58.63687 167.7495) (end 60.96887 165.4175) (width 0.25) (layer F.Cu) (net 8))
 (segment (start 60.96887 165.4175) (end 66.1035 165.4175) (width 0.25) (layer F.Cu) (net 8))
 (segment (start 73.3625 172.593) (end 75.3945 174.625) (width 0.25) (layer F.Cu) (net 8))
 (segment (start 57.5055 167.7495) (end 58.63687 167.7495) (width 0.25) (layer F.Cu) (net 8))
 (segment (start 66.1035 165.4175) (end 67.056 166.37) (width 0.25) (layer F.Cu) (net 8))
 (segment (start 39.4135 184.3405) (end 40.112 185.039) (width 0.25) (layer F.Cu) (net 10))
 (segment (start 38.1635 184.3405) (end 39.4135 184.3405) (width 0.25) (layer F.Cu) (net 10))
 (via (at 48.7045 184.658) (size 0.8) (drill 0.4) (layers F.Cu B.Cu) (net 10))
 (segment (start 48.3235 185.039) (end 48.7045 184.658) (width 0.25) (layer F.Cu) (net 10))
 (segment (start 40.112 185.039) (end 48.3235 185.039) (width 0.25) (layer F.Cu) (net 10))
 (segment (start 56.705501 173.629499) (end 57.5055 172.8295) (width 0.25) (layer B.Cu) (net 10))
 (segment (start 49.104499 181.230501) (end 56.705501 173.629499) (width 0.25) (layer B.Cu) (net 10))
 (segment (start 49.104499 184.258001) (end 49.104499 181.230501) (width 0.25) (layer B.Cu) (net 10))
 (segment (start 48.7045 184.658) (end 49.104499 184.258001) (width 0.25) (layer B.Cu) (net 10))
 (segment (start 61.468 179.332) (end 61.468 184.277) (width 0.25) (layer F.Cu) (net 11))
 (segment (start 57.5055 175.3695) (end 61.468 179.332) (width 0.25) (layer F.Cu) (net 11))
 (segment (start 31.095 160.782) (end 31.6665 161.3535) (width 0.25) (layer F.Cu) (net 12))
 (segment (start 29.845 160.782) (end 31.095 160.782) (width 0.25) (layer F.Cu) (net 12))
 (segment (start 42.614502 161.3535) (end 54.61 173.348998) (width 0.25) (layer F.Cu) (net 12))
 (segment (start 31.6665 161.3535) (end 42.614502 161.3535) (width 0.25) (layer F.Cu) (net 12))
 (segment (start 54.61 175.014) (end 57.5055 177.9095) (width 0.25) (layer F.Cu) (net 12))
 (segment (start 54.61 173.348998) (end 54.61 175.014) (width 0.25) (layer F.Cu) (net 12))
 (segment (start 31.095 174.879) (end 39.0325 182.8165) (width 0.25) (layer F.Cu) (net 13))
 (segment (start 29.845 174.879) (end 31.095 174.879) (width 0.25) (layer F.Cu) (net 13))
 (segment (start 55.1385 182.8165) (end 57.5055 180.4495) (width 0.25) (layer F.Cu) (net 13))
 (segment (start 39.0325 182.8165) (end 55.1385 182.8165) (width 0.25) (layer F.Cu) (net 13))
 (segment (start 24.0465 167.7035) (end 28.174 171.831) (width 0.25) (layer F.Cu) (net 14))
 (segment (start 22.7965 167.7035) (end 24.0465 167.7035) (width 0.25) (layer F.Cu) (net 14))
 (segment (start 33.647 171.831) (end 42.2655 180.4495) (width 0.25) (layer F.Cu) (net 14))
 (segment (start 28.174 171.831) (end 33.647 171.831) (width 0.25) (layer F.Cu) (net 14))
 (segment (start 36.7665 172.4105) (end 42.2655 177.9095) (width 0.25) (layer F.Cu) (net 15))
 (segment (start 36.7665 167.64) (end 36.7665 172.4105) (width 0.25) (layer F.Cu) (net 15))
 (segment (start 42.2655 175.3695) (end 38.862 171.966) (width 0.25) (layer F.Cu) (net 16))
 (segment (start 38.862 171.966) (end 38.862 166.3065) (width 0.25) (layer F.Cu) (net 16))
 (segment (start 38.862 166.3065) (end 35.814 163.2585) (width 0.25) (layer F.Cu) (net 16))
 (segment (start 35.814 163.2585) (end 28.6385 163.2585) (width 0.25) (layer F.Cu) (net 16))
 (segment (start 28.6385 163.2585) (end 26.416 161.036) (width 0.25) (layer F.Cu) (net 16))
 (segment (start 26.416 158.1785) (end 20.1295 151.892) (width 0.25) (layer F.Cu) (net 16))
 (segment (start 26.416 161.036) (end 26.416 158.1785) (width 0.25) (layer F.Cu) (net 16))
 (segment (start 78.105 151.892) (end 73.66 156.337) (width 0.25) (layer F.Cu) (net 17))
 (segment (start 73.66 156.337) (end 66.929 156.337) (width 0.25) (layer F.Cu) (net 17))
 (segment (start 66.929 156.337) (end 60.452 149.86) (width 0.25) (layer F.Cu) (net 17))
 (segment (start 60.452 149.86) (end 55.6895 149.86) (width 0.25) (layer F.Cu) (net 17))
 (segment (start 48.3235 157.226) (end 48.3235 162.814) (width 0.25) (layer F.Cu) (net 17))
 (via (at 48.3235 162.814) (size 0.8) (drill 0.4) (layers F.Cu B.Cu) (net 17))
 (segment (start 55.6895 149.86) (end 48.3235 157.226) (width 0.25) (layer F.Cu) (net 17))
 (segment (start 47.923501 167.171499) (end 43.065499 172.029501) (width 0.25) (layer B.Cu) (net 17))
 (segment (start 43.065499 172.029501) (end 42.2655 172.8295) (width 0.25) (layer B.Cu) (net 17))
 (segment (start 47.923501 163.213999) (end 47.923501 167.171499) (width 0.25) (layer B.Cu) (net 17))
 (segment (start 48.3235 162.814) (end 47.923501 163.213999) (width 0.25) (layer B.Cu) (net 17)))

